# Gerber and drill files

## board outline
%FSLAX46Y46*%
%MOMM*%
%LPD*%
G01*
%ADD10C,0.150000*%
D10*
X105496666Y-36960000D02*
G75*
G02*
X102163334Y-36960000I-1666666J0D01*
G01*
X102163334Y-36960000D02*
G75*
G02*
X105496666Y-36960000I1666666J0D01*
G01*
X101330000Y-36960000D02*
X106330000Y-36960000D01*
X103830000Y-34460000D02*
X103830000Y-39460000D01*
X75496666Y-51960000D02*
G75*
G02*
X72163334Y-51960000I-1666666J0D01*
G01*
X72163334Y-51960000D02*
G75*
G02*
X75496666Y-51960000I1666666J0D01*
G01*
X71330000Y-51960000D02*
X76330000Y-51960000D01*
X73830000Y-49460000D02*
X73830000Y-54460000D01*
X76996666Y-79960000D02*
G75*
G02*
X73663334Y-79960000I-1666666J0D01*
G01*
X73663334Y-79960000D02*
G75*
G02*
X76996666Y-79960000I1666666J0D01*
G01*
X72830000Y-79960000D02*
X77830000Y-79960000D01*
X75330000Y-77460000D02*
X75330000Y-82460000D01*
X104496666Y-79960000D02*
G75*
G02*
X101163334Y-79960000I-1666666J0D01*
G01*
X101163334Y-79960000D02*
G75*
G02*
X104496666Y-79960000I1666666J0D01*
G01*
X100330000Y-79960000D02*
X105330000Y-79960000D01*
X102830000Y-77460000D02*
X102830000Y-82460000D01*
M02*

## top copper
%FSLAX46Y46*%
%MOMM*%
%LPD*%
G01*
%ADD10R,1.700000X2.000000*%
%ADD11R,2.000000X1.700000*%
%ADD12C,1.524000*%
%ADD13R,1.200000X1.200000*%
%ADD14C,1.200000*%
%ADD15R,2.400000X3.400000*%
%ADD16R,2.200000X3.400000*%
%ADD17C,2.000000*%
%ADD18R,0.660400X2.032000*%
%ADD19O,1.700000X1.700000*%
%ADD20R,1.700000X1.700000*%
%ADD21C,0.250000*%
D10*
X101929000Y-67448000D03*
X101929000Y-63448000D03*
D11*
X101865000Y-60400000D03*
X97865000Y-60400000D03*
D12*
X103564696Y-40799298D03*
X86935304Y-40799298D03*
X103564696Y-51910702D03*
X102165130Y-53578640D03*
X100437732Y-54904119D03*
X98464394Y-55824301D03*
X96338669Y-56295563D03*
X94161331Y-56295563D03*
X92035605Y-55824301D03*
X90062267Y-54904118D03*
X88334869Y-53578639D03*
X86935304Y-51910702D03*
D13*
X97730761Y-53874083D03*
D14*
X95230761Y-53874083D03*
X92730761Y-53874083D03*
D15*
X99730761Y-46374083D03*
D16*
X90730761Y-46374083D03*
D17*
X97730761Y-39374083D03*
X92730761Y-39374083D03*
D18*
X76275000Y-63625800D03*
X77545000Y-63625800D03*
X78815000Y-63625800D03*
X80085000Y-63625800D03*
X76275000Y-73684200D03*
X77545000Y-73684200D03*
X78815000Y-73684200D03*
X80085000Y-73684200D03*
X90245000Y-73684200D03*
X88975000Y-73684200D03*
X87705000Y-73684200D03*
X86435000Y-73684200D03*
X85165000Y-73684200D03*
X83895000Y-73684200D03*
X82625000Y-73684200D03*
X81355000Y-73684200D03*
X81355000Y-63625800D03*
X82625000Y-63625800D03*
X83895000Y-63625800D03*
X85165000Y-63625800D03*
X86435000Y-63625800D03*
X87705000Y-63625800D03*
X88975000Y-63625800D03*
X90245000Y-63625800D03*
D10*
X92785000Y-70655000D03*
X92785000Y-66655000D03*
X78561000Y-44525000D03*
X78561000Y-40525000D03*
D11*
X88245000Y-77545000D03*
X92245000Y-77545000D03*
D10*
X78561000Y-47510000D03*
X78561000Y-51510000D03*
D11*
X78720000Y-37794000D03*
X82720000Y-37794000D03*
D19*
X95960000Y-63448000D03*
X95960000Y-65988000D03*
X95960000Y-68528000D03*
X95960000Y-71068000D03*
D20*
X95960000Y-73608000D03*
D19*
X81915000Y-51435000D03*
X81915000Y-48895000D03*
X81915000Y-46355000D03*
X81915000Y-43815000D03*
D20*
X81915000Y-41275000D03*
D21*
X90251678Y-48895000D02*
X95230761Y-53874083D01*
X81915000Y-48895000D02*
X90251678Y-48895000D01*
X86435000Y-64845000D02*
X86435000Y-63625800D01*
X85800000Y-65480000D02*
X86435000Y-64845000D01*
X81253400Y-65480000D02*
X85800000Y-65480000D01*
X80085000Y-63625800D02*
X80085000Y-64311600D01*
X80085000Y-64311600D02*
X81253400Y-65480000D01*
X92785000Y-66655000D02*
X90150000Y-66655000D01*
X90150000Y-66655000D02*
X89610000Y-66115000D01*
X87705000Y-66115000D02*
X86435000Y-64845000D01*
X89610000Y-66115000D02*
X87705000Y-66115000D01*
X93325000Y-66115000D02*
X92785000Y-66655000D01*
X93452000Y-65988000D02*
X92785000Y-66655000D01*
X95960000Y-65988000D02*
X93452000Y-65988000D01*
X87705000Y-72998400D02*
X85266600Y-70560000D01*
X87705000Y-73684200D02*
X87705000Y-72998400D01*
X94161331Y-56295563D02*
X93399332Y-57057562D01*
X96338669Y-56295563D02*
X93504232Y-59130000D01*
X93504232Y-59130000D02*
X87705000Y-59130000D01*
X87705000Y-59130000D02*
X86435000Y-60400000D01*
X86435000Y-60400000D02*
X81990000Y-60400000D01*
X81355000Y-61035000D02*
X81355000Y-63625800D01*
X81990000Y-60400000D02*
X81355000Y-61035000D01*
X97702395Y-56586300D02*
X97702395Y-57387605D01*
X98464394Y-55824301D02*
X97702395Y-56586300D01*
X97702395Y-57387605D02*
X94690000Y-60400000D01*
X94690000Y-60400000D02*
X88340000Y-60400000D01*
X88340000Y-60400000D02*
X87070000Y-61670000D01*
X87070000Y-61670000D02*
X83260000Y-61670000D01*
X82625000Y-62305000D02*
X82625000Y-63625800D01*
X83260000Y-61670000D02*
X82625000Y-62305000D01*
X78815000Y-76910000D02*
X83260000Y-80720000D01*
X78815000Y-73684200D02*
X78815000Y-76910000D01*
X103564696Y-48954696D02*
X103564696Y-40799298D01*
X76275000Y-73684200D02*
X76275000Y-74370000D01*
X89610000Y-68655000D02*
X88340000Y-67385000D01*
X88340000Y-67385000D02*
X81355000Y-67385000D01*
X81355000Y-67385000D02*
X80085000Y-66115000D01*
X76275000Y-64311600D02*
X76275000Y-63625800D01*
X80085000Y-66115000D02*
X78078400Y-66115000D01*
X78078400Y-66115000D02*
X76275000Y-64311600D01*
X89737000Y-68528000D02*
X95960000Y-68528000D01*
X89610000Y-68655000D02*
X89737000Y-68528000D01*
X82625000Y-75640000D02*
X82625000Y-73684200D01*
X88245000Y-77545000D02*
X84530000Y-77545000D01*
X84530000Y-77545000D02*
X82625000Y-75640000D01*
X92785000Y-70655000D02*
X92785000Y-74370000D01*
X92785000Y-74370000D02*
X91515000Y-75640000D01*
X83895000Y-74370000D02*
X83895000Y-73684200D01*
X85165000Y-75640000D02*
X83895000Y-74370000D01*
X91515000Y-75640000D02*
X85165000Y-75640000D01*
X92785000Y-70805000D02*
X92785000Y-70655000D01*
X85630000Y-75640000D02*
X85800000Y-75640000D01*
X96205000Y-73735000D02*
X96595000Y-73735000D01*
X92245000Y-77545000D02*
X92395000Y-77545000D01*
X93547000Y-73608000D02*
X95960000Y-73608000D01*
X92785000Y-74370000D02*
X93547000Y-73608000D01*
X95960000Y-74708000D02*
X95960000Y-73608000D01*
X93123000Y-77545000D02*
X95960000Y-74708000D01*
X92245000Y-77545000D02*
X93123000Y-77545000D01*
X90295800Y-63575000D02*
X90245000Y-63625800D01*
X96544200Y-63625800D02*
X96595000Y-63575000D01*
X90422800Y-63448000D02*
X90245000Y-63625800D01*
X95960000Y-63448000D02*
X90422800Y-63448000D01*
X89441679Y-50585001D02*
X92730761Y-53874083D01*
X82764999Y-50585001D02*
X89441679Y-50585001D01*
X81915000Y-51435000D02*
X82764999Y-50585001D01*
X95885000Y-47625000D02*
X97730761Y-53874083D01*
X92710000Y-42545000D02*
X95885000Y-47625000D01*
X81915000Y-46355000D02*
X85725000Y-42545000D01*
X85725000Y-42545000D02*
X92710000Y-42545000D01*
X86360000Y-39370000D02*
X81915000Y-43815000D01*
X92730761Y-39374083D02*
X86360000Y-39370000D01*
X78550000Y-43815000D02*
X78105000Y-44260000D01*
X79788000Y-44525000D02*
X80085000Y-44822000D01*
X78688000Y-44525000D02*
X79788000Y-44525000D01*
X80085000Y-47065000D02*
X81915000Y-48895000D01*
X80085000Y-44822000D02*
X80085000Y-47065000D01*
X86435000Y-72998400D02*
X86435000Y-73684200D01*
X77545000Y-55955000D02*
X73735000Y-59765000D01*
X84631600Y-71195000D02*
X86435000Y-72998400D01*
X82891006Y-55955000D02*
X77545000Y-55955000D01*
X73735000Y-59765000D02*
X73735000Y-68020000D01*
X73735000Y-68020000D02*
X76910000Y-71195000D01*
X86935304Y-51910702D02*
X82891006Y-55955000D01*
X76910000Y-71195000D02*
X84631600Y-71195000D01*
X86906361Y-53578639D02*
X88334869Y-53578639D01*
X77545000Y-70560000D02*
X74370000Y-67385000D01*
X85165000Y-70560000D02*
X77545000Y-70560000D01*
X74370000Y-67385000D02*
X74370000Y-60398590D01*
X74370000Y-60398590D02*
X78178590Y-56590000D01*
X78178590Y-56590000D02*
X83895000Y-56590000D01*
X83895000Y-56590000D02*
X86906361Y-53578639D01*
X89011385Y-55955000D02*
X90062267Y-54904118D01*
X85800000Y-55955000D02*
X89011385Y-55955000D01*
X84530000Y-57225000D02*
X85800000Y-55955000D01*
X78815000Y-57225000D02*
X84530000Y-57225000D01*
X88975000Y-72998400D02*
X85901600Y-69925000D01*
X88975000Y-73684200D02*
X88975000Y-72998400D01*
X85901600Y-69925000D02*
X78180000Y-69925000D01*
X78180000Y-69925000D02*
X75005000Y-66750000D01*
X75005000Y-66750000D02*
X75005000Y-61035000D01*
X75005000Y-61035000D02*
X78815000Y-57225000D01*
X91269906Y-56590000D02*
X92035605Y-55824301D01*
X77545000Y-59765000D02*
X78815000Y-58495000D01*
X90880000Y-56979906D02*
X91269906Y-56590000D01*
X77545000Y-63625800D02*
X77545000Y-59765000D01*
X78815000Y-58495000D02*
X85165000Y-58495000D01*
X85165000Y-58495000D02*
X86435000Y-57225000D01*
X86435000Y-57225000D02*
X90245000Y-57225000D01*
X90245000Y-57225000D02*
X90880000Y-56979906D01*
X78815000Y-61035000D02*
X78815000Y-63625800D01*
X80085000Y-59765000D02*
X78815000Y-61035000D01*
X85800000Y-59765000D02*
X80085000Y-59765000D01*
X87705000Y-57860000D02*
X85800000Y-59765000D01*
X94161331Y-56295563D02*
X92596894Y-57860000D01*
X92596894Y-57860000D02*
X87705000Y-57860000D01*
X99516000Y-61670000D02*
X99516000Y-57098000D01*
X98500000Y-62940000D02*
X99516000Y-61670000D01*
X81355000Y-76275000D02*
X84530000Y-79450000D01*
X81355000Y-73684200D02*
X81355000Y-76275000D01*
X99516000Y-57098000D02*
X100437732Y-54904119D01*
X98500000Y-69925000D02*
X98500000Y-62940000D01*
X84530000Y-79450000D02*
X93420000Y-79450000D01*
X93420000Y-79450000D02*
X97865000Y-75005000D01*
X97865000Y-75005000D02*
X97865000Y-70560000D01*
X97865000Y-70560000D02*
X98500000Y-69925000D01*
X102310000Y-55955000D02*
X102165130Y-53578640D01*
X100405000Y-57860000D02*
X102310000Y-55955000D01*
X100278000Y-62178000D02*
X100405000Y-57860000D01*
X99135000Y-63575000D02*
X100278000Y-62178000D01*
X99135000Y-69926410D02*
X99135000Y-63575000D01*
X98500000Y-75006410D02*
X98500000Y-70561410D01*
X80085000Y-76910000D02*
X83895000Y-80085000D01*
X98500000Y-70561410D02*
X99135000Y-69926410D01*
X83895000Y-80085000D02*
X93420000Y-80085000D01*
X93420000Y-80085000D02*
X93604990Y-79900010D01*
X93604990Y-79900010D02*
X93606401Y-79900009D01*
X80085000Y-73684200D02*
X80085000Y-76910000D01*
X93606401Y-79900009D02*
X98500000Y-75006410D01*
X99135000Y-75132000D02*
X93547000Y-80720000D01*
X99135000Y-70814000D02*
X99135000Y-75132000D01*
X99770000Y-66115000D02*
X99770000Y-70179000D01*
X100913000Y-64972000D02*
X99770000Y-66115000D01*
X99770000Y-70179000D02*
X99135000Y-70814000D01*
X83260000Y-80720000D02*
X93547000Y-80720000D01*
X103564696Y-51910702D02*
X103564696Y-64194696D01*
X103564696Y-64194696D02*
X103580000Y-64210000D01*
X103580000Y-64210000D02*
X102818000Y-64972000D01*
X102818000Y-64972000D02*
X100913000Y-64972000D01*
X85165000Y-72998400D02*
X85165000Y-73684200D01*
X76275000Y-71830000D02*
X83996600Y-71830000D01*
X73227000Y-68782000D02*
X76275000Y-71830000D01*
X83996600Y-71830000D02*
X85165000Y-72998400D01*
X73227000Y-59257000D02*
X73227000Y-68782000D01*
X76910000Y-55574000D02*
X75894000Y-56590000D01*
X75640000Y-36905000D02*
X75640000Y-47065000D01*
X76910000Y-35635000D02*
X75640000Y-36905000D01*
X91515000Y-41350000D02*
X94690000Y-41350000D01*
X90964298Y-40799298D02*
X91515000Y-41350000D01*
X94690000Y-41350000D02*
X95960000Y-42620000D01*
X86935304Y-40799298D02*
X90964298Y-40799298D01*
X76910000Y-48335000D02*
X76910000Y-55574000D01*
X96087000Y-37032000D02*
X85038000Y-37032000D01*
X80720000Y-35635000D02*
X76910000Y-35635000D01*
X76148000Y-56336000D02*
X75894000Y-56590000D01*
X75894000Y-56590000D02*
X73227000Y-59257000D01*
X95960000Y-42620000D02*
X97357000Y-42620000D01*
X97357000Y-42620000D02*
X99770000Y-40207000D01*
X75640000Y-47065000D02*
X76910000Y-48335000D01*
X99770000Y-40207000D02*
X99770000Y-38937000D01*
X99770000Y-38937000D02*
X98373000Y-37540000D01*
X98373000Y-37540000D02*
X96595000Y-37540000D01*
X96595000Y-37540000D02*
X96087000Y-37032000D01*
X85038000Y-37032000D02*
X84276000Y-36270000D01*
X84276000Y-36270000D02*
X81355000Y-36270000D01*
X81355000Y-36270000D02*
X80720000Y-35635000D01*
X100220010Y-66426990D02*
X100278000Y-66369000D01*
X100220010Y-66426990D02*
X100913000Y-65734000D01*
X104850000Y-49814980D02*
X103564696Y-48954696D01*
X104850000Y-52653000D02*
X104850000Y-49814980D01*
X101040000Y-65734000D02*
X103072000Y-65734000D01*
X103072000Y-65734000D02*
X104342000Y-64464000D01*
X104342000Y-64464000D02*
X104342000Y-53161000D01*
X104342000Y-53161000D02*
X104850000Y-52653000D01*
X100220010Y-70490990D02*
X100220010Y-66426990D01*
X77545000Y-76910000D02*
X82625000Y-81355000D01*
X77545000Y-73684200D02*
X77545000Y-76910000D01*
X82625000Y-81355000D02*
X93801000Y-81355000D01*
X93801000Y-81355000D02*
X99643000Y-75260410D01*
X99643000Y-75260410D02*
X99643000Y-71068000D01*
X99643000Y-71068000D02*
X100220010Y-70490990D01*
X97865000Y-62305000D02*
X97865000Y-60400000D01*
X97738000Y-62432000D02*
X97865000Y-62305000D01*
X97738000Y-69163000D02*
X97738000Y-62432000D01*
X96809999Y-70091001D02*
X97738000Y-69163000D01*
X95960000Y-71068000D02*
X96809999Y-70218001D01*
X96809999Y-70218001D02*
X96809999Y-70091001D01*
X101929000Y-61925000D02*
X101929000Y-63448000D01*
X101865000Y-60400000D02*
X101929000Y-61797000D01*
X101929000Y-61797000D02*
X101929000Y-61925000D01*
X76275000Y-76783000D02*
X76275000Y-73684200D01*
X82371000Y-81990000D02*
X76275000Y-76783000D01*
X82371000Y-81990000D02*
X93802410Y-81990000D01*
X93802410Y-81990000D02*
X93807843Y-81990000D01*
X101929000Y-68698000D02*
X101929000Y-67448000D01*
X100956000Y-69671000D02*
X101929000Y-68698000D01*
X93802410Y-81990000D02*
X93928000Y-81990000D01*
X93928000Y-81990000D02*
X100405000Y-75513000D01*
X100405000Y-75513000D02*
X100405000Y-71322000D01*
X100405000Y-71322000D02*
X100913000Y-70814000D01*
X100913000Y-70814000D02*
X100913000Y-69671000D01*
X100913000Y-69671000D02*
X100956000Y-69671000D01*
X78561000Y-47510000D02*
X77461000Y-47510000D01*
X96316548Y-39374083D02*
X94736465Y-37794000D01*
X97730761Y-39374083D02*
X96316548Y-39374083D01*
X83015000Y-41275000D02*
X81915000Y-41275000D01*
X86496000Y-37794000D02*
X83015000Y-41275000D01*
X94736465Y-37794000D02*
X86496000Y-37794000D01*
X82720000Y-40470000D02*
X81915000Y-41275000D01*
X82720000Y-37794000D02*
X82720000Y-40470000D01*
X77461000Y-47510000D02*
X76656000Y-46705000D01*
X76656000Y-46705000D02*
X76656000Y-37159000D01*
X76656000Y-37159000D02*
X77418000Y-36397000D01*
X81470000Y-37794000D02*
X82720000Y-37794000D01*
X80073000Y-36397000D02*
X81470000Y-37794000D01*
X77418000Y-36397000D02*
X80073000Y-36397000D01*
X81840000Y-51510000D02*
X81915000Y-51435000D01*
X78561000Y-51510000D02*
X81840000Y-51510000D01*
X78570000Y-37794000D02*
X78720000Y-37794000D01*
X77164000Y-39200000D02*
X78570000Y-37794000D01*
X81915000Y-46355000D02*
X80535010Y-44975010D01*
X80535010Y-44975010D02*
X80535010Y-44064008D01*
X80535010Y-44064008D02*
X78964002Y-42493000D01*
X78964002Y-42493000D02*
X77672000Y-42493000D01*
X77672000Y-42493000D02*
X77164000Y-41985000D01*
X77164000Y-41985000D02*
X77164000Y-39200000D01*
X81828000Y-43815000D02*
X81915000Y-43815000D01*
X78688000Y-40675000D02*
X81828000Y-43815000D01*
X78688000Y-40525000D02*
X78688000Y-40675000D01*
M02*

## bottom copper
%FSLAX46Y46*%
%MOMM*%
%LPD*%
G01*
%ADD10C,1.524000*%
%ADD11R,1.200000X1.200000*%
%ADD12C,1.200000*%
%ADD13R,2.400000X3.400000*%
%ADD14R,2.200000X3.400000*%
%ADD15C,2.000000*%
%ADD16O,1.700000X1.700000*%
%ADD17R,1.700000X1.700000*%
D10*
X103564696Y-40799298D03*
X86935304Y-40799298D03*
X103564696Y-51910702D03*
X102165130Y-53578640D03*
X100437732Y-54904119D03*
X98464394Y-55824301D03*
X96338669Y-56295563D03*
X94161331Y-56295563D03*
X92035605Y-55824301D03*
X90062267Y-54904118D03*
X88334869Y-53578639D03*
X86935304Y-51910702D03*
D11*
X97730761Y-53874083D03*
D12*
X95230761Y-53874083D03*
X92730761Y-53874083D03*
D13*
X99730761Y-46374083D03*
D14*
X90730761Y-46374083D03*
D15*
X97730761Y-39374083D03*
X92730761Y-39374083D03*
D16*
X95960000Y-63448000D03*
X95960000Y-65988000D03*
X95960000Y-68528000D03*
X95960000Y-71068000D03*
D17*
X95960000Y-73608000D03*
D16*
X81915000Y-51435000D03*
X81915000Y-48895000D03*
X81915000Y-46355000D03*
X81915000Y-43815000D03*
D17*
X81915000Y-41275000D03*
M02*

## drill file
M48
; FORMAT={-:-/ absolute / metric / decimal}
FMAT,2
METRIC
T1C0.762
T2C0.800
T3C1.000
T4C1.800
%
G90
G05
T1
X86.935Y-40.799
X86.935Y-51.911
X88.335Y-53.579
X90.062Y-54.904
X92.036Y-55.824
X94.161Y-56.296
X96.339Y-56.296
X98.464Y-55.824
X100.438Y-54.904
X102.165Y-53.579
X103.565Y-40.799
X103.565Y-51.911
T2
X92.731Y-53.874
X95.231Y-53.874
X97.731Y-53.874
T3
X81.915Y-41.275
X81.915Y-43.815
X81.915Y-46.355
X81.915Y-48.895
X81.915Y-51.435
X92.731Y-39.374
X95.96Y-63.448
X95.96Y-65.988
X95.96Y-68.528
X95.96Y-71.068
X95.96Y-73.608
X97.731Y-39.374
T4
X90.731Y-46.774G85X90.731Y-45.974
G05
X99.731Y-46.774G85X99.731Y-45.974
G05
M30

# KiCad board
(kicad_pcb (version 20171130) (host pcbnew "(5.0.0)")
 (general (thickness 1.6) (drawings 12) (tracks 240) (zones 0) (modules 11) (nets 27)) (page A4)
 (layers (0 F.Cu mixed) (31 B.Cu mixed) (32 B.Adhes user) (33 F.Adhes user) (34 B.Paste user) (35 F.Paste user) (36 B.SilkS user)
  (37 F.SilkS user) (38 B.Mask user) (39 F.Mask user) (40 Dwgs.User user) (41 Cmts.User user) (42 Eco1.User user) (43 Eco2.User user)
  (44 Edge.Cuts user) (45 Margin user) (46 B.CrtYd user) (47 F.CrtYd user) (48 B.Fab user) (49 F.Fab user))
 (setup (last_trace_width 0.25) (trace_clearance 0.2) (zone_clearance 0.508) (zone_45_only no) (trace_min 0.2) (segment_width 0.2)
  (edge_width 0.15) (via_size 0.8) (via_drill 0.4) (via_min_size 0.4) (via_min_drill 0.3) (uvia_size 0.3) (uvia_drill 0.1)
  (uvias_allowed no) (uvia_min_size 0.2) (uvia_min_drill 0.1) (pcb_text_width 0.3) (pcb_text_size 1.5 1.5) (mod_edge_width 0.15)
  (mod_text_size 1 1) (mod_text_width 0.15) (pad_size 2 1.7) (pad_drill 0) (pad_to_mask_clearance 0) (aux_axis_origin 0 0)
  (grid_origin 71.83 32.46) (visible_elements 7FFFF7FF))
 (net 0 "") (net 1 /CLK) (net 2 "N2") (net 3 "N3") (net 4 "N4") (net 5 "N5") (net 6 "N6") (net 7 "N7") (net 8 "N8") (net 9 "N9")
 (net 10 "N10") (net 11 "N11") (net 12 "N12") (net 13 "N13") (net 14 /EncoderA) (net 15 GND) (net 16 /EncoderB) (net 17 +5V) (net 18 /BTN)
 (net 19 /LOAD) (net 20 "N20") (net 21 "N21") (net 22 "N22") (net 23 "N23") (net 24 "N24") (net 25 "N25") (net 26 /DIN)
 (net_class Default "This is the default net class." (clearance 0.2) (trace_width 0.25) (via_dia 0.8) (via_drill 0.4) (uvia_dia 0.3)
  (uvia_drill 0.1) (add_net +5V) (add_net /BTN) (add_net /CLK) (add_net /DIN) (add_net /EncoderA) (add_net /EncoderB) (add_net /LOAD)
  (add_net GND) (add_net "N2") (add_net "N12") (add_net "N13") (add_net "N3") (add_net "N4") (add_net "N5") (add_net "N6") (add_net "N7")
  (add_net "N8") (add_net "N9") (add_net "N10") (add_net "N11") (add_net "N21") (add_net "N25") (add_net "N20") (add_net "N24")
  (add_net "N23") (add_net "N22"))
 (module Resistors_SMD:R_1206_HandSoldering (layer F.Cu) (at 101.929 65.448 90)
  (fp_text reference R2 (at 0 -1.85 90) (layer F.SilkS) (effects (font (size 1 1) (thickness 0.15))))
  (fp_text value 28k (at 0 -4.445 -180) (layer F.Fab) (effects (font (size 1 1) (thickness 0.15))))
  (pad 1 smd rect (at -2 0 90) (size 2 1.7) (layers F.Cu F.Paste F.Mask) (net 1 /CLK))
  (pad 2 smd rect (at 2 0 90) (size 2 1.7) (layers F.Cu F.Paste F.Mask) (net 1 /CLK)))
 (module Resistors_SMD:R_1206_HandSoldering (layer F.Cu) (at 99.865 60.4)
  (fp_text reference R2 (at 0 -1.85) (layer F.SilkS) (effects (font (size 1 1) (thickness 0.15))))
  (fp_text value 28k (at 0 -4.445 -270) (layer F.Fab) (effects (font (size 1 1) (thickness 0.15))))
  (pad 2 smd rect (at 2 0) (size 2 1.7) (layers F.Cu F.Paste F.Mask) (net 1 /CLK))
  (pad 1 smd rect (at -2 0) (size 2 1.7) (layers F.Cu F.Paste F.Mask) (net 1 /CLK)))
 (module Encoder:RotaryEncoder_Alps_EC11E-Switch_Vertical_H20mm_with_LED (layer B.Cu) (at 95.25 46.355 180)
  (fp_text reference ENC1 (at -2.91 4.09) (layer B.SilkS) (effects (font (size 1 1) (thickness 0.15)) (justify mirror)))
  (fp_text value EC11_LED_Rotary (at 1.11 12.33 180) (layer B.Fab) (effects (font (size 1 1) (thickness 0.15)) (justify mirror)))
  (pad 1 thru_hole circle (at -8.314696 5.555702 123.8) (size 1.524 1.524) (drill 0.762) (layers *.Cu *.Mask) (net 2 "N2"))
  (pad 12 thru_hole circle (at 8.314696 5.555702 123.8) (size 1.524 1.524) (drill 0.762) (layers *.Cu *.Mask) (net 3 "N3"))
  (pad 2 thru_hole circle (at -8.314696 -5.555702 123.8) (size 1.524 1.524) (drill 0.762) (layers *.Cu *.Mask) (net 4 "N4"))
  (pad 3 thru_hole circle (at -6.91513 -7.22364 123.8) (size 1.524 1.524) (drill 0.762) (layers *.Cu *.Mask) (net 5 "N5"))
  (pad 4 thru_hole circle (at -5.187732 -8.549119 123.8) (size 1.524 1.524) (drill 0.762) (layers *.Cu *.Mask) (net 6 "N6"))
  (pad 5 thru_hole circle (at -3.214394 -9.469301 123.8) (size 1.524 1.524) (drill 0.762) (layers *.Cu *.Mask) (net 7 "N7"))
  (pad 6 thru_hole circle (at -1.088669 -9.940563 123.8) (size 1.524 1.524) (drill 0.762) (layers *.Cu *.Mask) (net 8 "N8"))
  (pad 7 thru_hole circle (at 1.088669 -9.940563 123.8) (size 1.524 1.524) (drill 0.762) (layers *.Cu *.Mask) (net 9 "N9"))
  (pad 8 thru_hole circle (at 3.214395 -9.469301 123.8) (size 1.524 1.524) (drill 0.762) (layers *.Cu *.Mask) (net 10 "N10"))
  (pad 9 thru_hole circle (at 5.187733 -8.549118 123.8) (size 1.524 1.524) (drill 0.762) (layers *.Cu *.Mask) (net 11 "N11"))
  (pad 10 thru_hole circle (at 6.915131 -7.223639 123.8) (size 1.524 1.524) (drill 0.762) (layers *.Cu *.Mask) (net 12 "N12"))
  (pad 11 thru_hole circle (at 8.314696 -5.555702 123.8) (size 1.524 1.524) (drill 0.762) (layers *.Cu *.Mask) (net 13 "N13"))
  (pad A thru_hole rect (at -2.480761 -7.519083 90) (size 1.2 1.2) (drill 0.8) (layers *.Cu *.Mask) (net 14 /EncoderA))
  (pad C thru_hole circle (at 0.019239 -7.519083 90) (size 1.2 1.2) (drill 0.8) (layers *.Cu *.Mask) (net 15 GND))
  (pad B thru_hole circle (at 2.519239 -7.519083 90) (size 1.2 1.2) (drill 0.8) (layers *.Cu *.Mask) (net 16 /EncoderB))
  (pad MP thru_hole rect (at -4.480761 -0.019083 90) (size 3.4 2.4) (drill oval 2.6 1.8) (layers *.Cu *.Mask))
  (pad MP thru_hole rect (at 4.519239 -0.019083 90) (size 3.4 2.2) (drill oval 2.6 1.8) (layers *.Cu *.Mask))
  (pad SW2 thru_hole circle (at -2.480761 6.980917 90) (size 2 2) (drill 1) (layers *.Cu *.Mask) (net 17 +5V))
  (pad SW1 thru_hole circle (at 2.519239 6.980917 90) (size 2 2) (drill 1) (layers *.Cu *.Mask) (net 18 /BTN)))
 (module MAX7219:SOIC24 (layer F.Cu) (at 83.26 68.655 180)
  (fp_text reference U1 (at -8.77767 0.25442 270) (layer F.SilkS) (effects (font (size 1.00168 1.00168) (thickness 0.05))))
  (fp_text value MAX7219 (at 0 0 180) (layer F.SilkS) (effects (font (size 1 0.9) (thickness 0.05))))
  (pad 12 smd rect (at 6.985 5.0292 180) (size 0.6604 2.032) (layers F.Cu F.Paste F.Mask) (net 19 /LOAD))
  (pad 11 smd rect (at 5.715 5.0292 180) (size 0.6604 2.032) (layers F.Cu F.Paste F.Mask) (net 10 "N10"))
  (pad 10 smd rect (at 4.445 5.0292 180) (size 0.6604 2.032) (layers F.Cu F.Paste F.Mask) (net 9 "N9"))
  (pad 9 smd rect (at 3.175 5.0292 180) (size 0.6604 2.032) (layers F.Cu F.Paste F.Mask) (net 15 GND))
  (pad 13 smd rect (at 6.985 -5.0292 180) (size 0.6604 2.032) (layers F.Cu F.Paste F.Mask) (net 1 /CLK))
  (pad 14 smd rect (at 5.715 -5.0292 180) (size 0.6604 2.032) (layers F.Cu F.Paste F.Mask) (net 2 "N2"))
  (pad 15 smd rect (at 4.445 -5.0292 180) (size 0.6604 2.032) (layers F.Cu F.Paste F.Mask) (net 4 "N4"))
  (pad 16 smd rect (at 3.175 -5.0292 180) (size 0.6604 2.032) (layers F.Cu F.Paste F.Mask) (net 5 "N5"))
  (pad 24 smd rect (at -6.985 -5.0292 180) (size 0.6604 2.032) (layers F.Cu F.Paste F.Mask) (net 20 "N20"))
  (pad 23 smd rect (at -5.715 -5.0292 180) (size 0.6604 2.032) (layers F.Cu F.Paste F.Mask) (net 11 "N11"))
  (pad 22 smd rect (at -4.445 -5.0292 180) (size 0.6604 2.032) (layers F.Cu F.Paste F.Mask) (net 12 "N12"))
  (pad 21 smd rect (at -3.175 -5.0292 180) (size 0.6604 2.032) (layers F.Cu F.Paste F.Mask) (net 13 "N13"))
  (pad 20 smd rect (at -1.905 -5.0292 180) (size 0.6604 2.032) (layers F.Cu F.Paste F.Mask) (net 3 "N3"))
  (pad 19 smd rect (at -0.635 -5.0292 180) (size 0.6604 2.032) (layers F.Cu F.Paste F.Mask) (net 17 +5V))
  (pad 18 smd rect (at 0.635 -5.0292 180) (size 0.6604 2.032) (layers F.Cu F.Paste F.Mask) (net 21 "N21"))
  (pad 17 smd rect (at 1.905 -5.0292 180) (size 0.6604 2.032) (layers F.Cu F.Paste F.Mask) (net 6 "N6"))
  (pad 8 smd rect (at 1.905 5.0292 180) (size 0.6604 2.032) (layers F.Cu F.Paste F.Mask) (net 8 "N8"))
  (pad 7 smd rect (at 0.635 5.0292 180) (size 0.6604 2.032) (layers F.Cu F.Paste F.Mask) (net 7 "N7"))
  (pad 6 smd rect (at -0.635 5.0292 180) (size 0.6604 2.032) (layers F.Cu F.Paste F.Mask) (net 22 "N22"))
  (pad 5 smd rect (at -1.905 5.0292 180) (size 0.6604 2.032) (layers F.Cu F.Paste F.Mask) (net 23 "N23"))
  (pad 4 smd rect (at -3.175 5.0292 180) (size 0.6604 2.032) (layers F.Cu F.Paste F.Mask) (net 15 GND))
  (pad 3 smd rect (at -4.445 5.0292 180) (size 0.6604 2.032) (layers F.Cu F.Paste F.Mask) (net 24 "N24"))
  (pad 2 smd rect (at -5.715 5.0292 180) (size 0.6604 2.032) (layers F.Cu F.Paste F.Mask) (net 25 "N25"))
  (pad 1 smd rect (at -6.985 5.0292 180) (size 0.6604 2.032) (layers F.Cu F.Paste F.Mask) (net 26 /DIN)))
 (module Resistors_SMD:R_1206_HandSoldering (layer F.Cu) (at 92.785 68.655 90)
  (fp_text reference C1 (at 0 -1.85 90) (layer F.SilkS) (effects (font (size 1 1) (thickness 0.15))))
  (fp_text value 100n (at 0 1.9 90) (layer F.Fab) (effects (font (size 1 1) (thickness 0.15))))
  (pad 1 smd rect (at -2 0 90) (size 2 1.7) (layers F.Cu F.Paste F.Mask) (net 17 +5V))
  (pad 2 smd rect (at 2 0 90) (size 2 1.7) (layers F.Cu F.Paste F.Mask) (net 15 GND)))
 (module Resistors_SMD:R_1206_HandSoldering (layer F.Cu) (at 78.561 42.525 90)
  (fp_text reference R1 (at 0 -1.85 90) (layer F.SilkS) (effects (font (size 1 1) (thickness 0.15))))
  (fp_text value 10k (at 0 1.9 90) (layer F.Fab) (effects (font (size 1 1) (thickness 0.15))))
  (pad 1 smd rect (at -2 0 90) (size 2 1.7) (layers F.Cu F.Paste F.Mask) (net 15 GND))
  (pad 2 smd rect (at 2 0 90) (size 2 1.7) (layers F.Cu F.Paste F.Mask) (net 18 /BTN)))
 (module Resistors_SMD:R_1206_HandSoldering (layer F.Cu) (at 90.245 77.545)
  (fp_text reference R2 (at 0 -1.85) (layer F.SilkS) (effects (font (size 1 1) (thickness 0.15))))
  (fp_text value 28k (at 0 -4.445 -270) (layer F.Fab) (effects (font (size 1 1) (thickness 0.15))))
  (pad 1 smd rect (at -2 0) (size 2 1.7) (layers F.Cu F.Paste F.Mask) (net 21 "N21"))
  (pad 2 smd rect (at 2 0) (size 2 1.7) (layers F.Cu F.Paste F.Mask) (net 17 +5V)))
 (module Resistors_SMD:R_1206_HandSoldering (layer F.Cu) (at 78.561 49.51 270)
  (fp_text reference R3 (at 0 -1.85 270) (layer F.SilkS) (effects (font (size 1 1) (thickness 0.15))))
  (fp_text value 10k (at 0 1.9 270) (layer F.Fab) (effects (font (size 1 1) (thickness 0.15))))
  (pad 1 smd rect (at -2 0 270) (size 2 1.7) (layers F.Cu F.Paste F.Mask) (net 17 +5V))
  (pad 2 smd rect (at 2 0 270) (size 2 1.7) (layers F.Cu F.Paste F.Mask) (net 16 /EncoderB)))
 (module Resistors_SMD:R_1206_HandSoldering (layer F.Cu) (at 80.72 37.794)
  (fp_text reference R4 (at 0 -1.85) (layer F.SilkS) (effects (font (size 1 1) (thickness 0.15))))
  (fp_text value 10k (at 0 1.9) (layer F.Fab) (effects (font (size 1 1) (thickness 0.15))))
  (pad 1 smd rect (at -2 0) (size 2 1.7) (layers F.Cu F.Paste F.Mask) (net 14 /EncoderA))
  (pad 2 smd rect (at 2 0) (size 2 1.7) (layers F.Cu F.Paste F.Mask) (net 17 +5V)))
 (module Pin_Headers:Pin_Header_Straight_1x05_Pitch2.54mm (layer F.Cu) (at 95.96 73.608 180)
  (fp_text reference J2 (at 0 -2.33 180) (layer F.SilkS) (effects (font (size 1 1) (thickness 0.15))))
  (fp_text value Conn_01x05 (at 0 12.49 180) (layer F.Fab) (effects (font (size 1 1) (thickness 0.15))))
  (pad 5 thru_hole oval (at 0 10.16 180) (size 1.7 1.7) (drill 1) (layers *.Cu *.Mask) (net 26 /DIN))
  (pad 4 thru_hole oval (at 0 7.62 180) (size 1.7 1.7) (drill 1) (layers *.Cu *.Mask) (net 15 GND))
  (pad 3 thru_hole oval (at 0 5.08 180) (size 1.7 1.7) (drill 1) (layers *.Cu *.Mask) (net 19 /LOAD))
  (pad 2 thru_hole oval (at 0 2.54 180) (size 1.7 1.7) (drill 1) (layers *.Cu *.Mask) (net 1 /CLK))
  (pad 1 thru_hole rect (at 0 0 180) (size 1.7 1.7) (drill 1) (layers *.Cu *.Mask) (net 17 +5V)))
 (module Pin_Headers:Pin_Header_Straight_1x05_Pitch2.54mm (layer F.Cu) (at 81.915 41.275)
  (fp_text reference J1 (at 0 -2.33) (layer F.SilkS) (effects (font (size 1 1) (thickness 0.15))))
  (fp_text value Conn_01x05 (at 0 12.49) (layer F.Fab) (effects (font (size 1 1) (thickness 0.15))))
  (pad 5 thru_hole oval (at 0 10.16) (size 1.7 1.7) (drill 1) (layers *.Cu *.Mask) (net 16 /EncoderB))
  (pad 4 thru_hole oval (at 0 7.62) (size 1.7 1.7) (drill 1) (layers *.Cu *.Mask) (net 15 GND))
  (pad 3 thru_hole oval (at 0 5.08) (size 1.7 1.7) (drill 1) (layers *.Cu *.Mask) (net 14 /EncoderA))
  (pad 2 thru_hole oval (at 0 2.54) (size 1.7 1.7) (drill 1) (layers *.Cu *.Mask) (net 18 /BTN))
  (pad 1 thru_hole rect (at 0 0) (size 1.7 1.7) (drill 1) (layers *.Cu *.Mask) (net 17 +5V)))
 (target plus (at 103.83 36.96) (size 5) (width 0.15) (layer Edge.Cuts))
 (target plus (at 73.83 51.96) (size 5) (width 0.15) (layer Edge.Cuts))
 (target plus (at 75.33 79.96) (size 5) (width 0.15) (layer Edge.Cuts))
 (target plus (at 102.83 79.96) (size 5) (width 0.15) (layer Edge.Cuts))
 (segment (start 90.251678 48.895) (end 95.230761 53.874083) (width 0.25) (layer F.Cu) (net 15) (status 20))
 (segment (start 81.915 48.895) (end 90.251678 48.895) (width 0.25) (layer F.Cu) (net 15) (status 10))
 (segment (start 86.435 64.845) (end 86.435 63.6258) (width 0.25) (layer F.Cu) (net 15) (status 20))
 (segment (start 85.8 65.48) (end 86.435 64.845) (width 0.25) (layer F.Cu) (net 15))
 (segment (start 81.2534 65.48) (end 85.8 65.48) (width 0.25) (layer F.Cu) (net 15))
 (segment (start 80.085 63.6258) (end 80.085 64.3116) (width 0.25) (layer F.Cu) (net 15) (status 30))
 (segment (start 80.085 64.3116) (end 81.2534 65.48) (width 0.25) (layer F.Cu) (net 15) (status 10))
 (segment (start 92.785 66.655) (end 90.15 66.655) (width 0.25) (layer F.Cu) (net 15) (status 10))
 (segment (start 90.15 66.655) (end 89.61 66.115) (width 0.25) (layer F.Cu) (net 15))
 (segment (start 87.705 66.115) (end 86.435 64.845) (width 0.25) (layer F.Cu) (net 15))
 (segment (start 89.61 66.115) (end 87.705 66.115) (width 0.25) (layer F.Cu) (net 15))
 (segment (start 93.325 66.115) (end 92.785 66.655) (width 0.25) (layer F.Cu) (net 15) (status 30))
 (segment (start 93.452 65.988) (end 92.785 66.655) (width 0.25) (layer F.Cu) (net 15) (status 30))
 (segment (start 95.96 65.988) (end 93.452 65.988) (width 0.25) (layer F.Cu) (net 15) (status 30))
 (segment (start 87.705 72.9984) (end 85.2666 70.56) (width 0.25) (layer F.Cu) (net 12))
 (segment (start 87.705 73.6842) (end 87.705 72.9984) (width 0.25) (layer F.Cu) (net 12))
 (segment (start 94.161331 56.295563) (end 93.399332 57.057562) (width 0.25) (layer F.Cu) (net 9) (status 10))
 (segment (start 96.338669 56.295563) (end 93.504232 59.13) (width 0.25) (layer F.Cu) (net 8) (status 10))
 (segment (start 93.504232 59.13) (end 87.705 59.13) (width 0.25) (layer F.Cu) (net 8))
 (segment (start 87.705 59.13) (end 86.435 60.4) (width 0.25) (layer F.Cu) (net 8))
 (segment (start 86.435 60.4) (end 81.99 60.4) (width 0.25) (layer F.Cu) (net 8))
 (segment (start 81.355 61.035) (end 81.355 63.6258) (width 0.25) (layer F.Cu) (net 8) (status 20))
 (segment (start 81.99 60.4) (end 81.355 61.035) (width 0.25) (layer F.Cu) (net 8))
 (segment (start 97.702395 56.5863) (end 97.702395 57.387605) (width 0.25) (layer F.Cu) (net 7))
 (segment (start 98.464394 55.824301) (end 97.702395 56.5863) (width 0.25) (layer F.Cu) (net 7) (status 10))
 (segment (start 97.702395 57.387605) (end 94.69 60.4) (width 0.25) (layer F.Cu) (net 7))
 (segment (start 94.69 60.4) (end 88.34 60.4) (width 0.25) (layer F.Cu) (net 7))
 (segment (start 88.34 60.4) (end 87.07 61.67) (width 0.25) (layer F.Cu) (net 7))
 (segment (start 87.07 61.67) (end 83.26 61.67) (width 0.25) (layer F.Cu) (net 7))
 (segment (start 82.625 62.305) (end 82.625 63.6258) (width 0.25) (layer F.Cu) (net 7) (status 20))
 (segment (start 83.26 61.67) (end 82.625 62.305) (width 0.25) (layer F.Cu) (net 7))
 (segment (start 78.815 76.91) (end 83.26 80.72) (width 0.25) (layer F.Cu) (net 4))
 (segment (start 78.815 73.6842) (end 78.815 76.91) (width 0.25) (layer F.Cu) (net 4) (status 10))
 (segment (start 103.564696 48.954696) (end 103.564696 40.799298) (width 0.25) (layer F.Cu) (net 2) (status 20))
 (segment (start 76.275 73.6842) (end 76.275 74.37) (width 0.25) (layer F.Cu) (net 1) (status 30))
 (segment (start 89.61 68.655) (end 88.34 67.385) (width 0.25) (layer F.Cu) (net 19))
 (segment (start 88.34 67.385) (end 81.355 67.385) (width 0.25) (layer F.Cu) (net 19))
 (segment (start 81.355 67.385) (end 80.085 66.115) (width 0.25) (layer F.Cu) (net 19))
 (segment (start 76.275 64.3116) (end 76.275 63.6258) (width 0.25) (layer F.Cu) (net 19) (status 30))
 (segment (start 80.085 66.115) (end 78.0784 66.115) (width 0.25) (layer F.Cu) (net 19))
 (segment (start 78.0784 66.115) (end 76.275 64.3116) (width 0.25) (layer F.Cu) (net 19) (status 20))
 (segment (start 89.737 68.528) (end 95.96 68.528) (width 0.25) (layer F.Cu) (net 19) (status 20))
 (segment (start 89.61 68.655) (end 89.737 68.528) (width 0.25) (layer F.Cu) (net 19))
 (segment (start 82.625 75.64) (end 82.625 73.6842) (width 0.25) (layer F.Cu) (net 21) (status 20))
 (segment (start 88.245 77.545) (end 84.53 77.545) (width 0.25) (layer F.Cu) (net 21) (status 10))
 (segment (start 84.53 77.545) (end 82.625 75.64) (width 0.25) (layer F.Cu) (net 21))
 (segment (start 92.785 70.655) (end 92.785 74.37) (width 0.25) (layer F.Cu) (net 17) (status 10))
 (segment (start 92.785 74.37) (end 91.515 75.64) (width 0.25) (layer F.Cu) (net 17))
 (segment (start 83.895 74.37) (end 83.895 73.6842) (width 0.25) (layer F.Cu) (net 17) (status 30))
 (segment (start 85.165 75.64) (end 83.895 74.37) (width 0.25) (layer F.Cu) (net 17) (status 20))
 (segment (start 91.515 75.64) (end 85.165 75.64) (width 0.25) (layer F.Cu) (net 17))
 (segment (start 92.785 70.805) (end 92.785 70.655) (width 0.25) (layer F.Cu) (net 17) (status 30))
 (segment (start 85.63 75.64) (end 85.8 75.64) (width 0.25) (layer F.Cu) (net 17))
 (segment (start 96.205 73.735) (end 96.595 73.735) (width 0.25) (layer F.Cu) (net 17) (status 30))
 (segment (start 92.245 77.545) (end 92.395 77.545) (width 0.25) (layer F.Cu) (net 17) (status 30))
 (segment (start 93.547 73.608) (end 95.96 73.608) (width 0.25) (layer F.Cu) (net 17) (status 20))
 (segment (start 92.785 74.37) (end 93.547 73.608) (width 0.25) (layer F.Cu) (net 17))
 (segment (start 95.96 74.708) (end 95.96 73.608) (width 0.25) (layer F.Cu) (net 17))
 (segment (start 93.123 77.545) (end 95.96 74.708) (width 0.25) (layer F.Cu) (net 17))
 (segment (start 92.245 77.545) (end 93.123 77.545) (width 0.25) (layer F.Cu) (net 17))
 (segment (start 90.2958 63.575) (end 90.245 63.6258) (width 0.25) (layer F.Cu) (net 26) (status 30))
 (segment (start 96.5442 63.6258) (end 96.595 63.575) (width 0.25) (layer F.Cu) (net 26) (status 30))
 (segment (start 90.4228 63.448) (end 90.245 63.6258) (width 0.25) (layer F.Cu) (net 26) (status 30))
 (segment (start 95.96 63.448) (end 90.4228 63.448) (width 0.25) (layer F.Cu) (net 26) (status 30))
 (segment (start 89.441679 50.585001) (end 92.730761 53.874083) (width 0.25) (layer F.Cu) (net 16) (status 20))
 (segment (start 82.764999 50.585001) (end 89.441679 50.585001) (width 0.25) (layer F.Cu) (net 16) (status 10))
 (segment (start 81.915 51.435) (end 82.764999 50.585001) (width 0.25) (layer F.Cu) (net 16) (status 30))
 (segment (start 95.885 47.625) (end 97.730761 53.874083) (width 0.25) (layer F.Cu) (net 14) (status 20))
 (segment (start 92.71 42.545) (end 95.885 47.625) (width 0.25) (layer F.Cu) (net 14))
 (segment (start 81.915 46.355) (end 85.725 42.545) (width 0.25) (layer F.Cu) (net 14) (status 10))
 (segment (start 85.725 42.545) (end 92.71 42.545) (width 0.25) (layer F.Cu) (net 14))
 (segment (start 86.36 39.37) (end 81.915 43.815) (width 0.25) (layer F.Cu) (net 18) (status 20))
 (segment (start 92.730761 39.374083) (end 86.36 39.37) (width 0.25) (layer F.Cu) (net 18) (status 10))
 (segment (start 78.55 43.815) (end 78.105 44.26) (width 0.25) (layer F.Cu) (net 15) (status 30))
 (segment (start 79.788 44.525) (end 80.085 44.822) (width 0.25) (layer F.Cu) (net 15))
 (segment (start 78.688 44.525) (end 79.788 44.525) (width 0.25) (layer F.Cu) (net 15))
 (segment (start 80.085 47.065) (end 81.915 48.895) (width 0.25) (layer F.Cu) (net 15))
 (segment (start 80.085 44.822) (end 80.085 47.065) (width 0.25) (layer F.Cu) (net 15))
 (segment (start 86.435 72.9984) (end 86.435 73.6842) (width 0.25) (layer F.Cu) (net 13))
 (segment (start 77.545 55.955) (end 73.735 59.765) (width 0.25) (layer F.Cu) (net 13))
 (segment (start 84.6316 71.195) (end 86.435 72.9984) (width 0.25) (layer F.Cu) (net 13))
 (segment (start 82.891006 55.955) (end 77.545 55.955) (width 0.25) (layer F.Cu) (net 13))
 (segment (start 73.735 59.765) (end 73.735 68.02) (width 0.25) (layer F.Cu) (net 13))
 (segment (start 73.735 68.02) (end 76.91 71.195) (width 0.25) (layer F.Cu) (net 13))
 (segment (start 86.935304 51.910702) (end 82.891006 55.955) (width 0.25) (layer F.Cu) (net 13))
 (segment (start 76.91 71.195) (end 84.6316 71.195) (width 0.25) (layer F.Cu) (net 13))
 (segment (start 86.906361 53.578639) (end 88.334869 53.578639) (width 0.25) (layer F.Cu) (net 12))
 (segment (start 77.545 70.56) (end 74.37 67.385) (width 0.25) (layer F.Cu) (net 12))
 (segment (start 85.165 70.56) (end 77.545 70.56) (width 0.25) (layer F.Cu) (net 12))
 (segment (start 74.37 67.385) (end 74.37 60.39859) (width 0.25) (layer F.Cu) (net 12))
 (segment (start 74.37 60.39859) (end 78.17859 56.59) (width 0.25) (layer F.Cu) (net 12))
 (segment (start 78.17859 56.59) (end 83.895 56.59) (width 0.25) (layer F.Cu) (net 12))
 (segment (start 83.895 56.59) (end 86.906361 53.578639) (width 0.25) (layer F.Cu) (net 12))
 (segment (start 89.011385 55.955) (end 90.062267 54.904118) (width 0.25) (layer F.Cu) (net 11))
 (segment (start 85.8 55.955) (end 89.011385 55.955) (width 0.25) (layer F.Cu) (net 11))
 (segment (start 84.53 57.225) (end 85.8 55.955) (width 0.25) (layer F.Cu) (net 11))
 (segment (start 78.815 57.225) (end 84.53 57.225) (width 0.25) (layer F.Cu) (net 11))
 (segment (start 88.975 72.9984) (end 85.9016 69.925) (width 0.25) (layer F.Cu) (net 11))
 (segment (start 88.975 73.6842) (end 88.975 72.9984) (width 0.25) (layer F.Cu) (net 11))
 (segment (start 85.9016 69.925) (end 78.18 69.925) (width 0.25) (layer F.Cu) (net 11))
 (segment (start 78.18 69.925) (end 75.005 66.75) (width 0.25) (layer F.Cu) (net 11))
 (segment (start 75.005 66.75) (end 75.005 61.035) (width 0.25) (layer F.Cu) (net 11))
 (segment (start 75.005 61.035) (end 78.815 57.225) (width 0.25) (layer F.Cu) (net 11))
 (segment (start 91.269906 56.59) (end 92.035605 55.824301) (width 0.25) (layer F.Cu) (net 10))
 (segment (start 77.545 59.765) (end 78.815 58.495) (width 0.25) (layer F.Cu) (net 10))
 (segment (start 90.88 56.979906) (end 91.269906 56.59) (width 0.25) (layer F.Cu) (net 10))
 (segment (start 77.545 63.6258) (end 77.545 59.765) (width 0.25) (layer F.Cu) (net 10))
 (segment (start 78.815 58.495) (end 85.165 58.495) (width 0.25) (layer F.Cu) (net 10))
 (segment (start 85.165 58.495) (end 86.435 57.225) (width 0.25) (layer F.Cu) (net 10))
 (segment (start 86.435 57.225) (end 90.245 57.225) (width 0.25) (layer F.Cu) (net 10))
 (segment (start 90.245 57.225) (end 90.88 56.979906) (width 0.25) (layer F.Cu) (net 10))
 (segment (start 78.815 61.035) (end 78.815 63.6258) (width 0.25) (layer F.Cu) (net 9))
 (segment (start 80.085 59.765) (end 78.815 61.035) (width 0.25) (layer F.Cu) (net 9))
 (segment (start 85.8 59.765) (end 80.085 59.765) (width 0.25) (layer F.Cu) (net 9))
 (segment (start 87.705 57.86) (end 85.8 59.765) (width 0.25) (layer F.Cu) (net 9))
 (segment (start 94.161331 56.295563) (end 92.596894 57.86) (width 0.25) (layer F.Cu) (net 9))
 (segment (start 92.596894 57.86) (end 87.705 57.86) (width 0.25) (layer F.Cu) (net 9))
 (segment (start 99.516 61.67) (end 99.516 57.098) (width 0.25) (layer F.Cu) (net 6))
 (segment (start 98.5 62.94) (end 99.516 61.67) (width 0.25) (layer F.Cu) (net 6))
 (segment (start 81.355 76.275) (end 84.53 79.45) (width 0.25) (layer F.Cu) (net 6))
 (segment (start 81.355 73.6842) (end 81.355 76.275) (width 0.25) (layer F.Cu) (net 6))
 (segment (start 99.516 57.098) (end 100.437732 54.904119) (width 0.25) (layer F.Cu) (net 6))
 (segment (start 98.5 69.925) (end 98.5 62.94) (width 0.25) (layer F.Cu) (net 6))
 (segment (start 84.53 79.45) (end 93.42 79.45) (width 0.25) (layer F.Cu) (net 6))
 (segment (start 93.42 79.45) (end 97.865 75.005) (width 0.25) (layer F.Cu) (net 6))
 (segment (start 97.865 75.005) (end 97.865 70.56) (width 0.25) (layer F.Cu) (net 6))
 (segment (start 97.865 70.56) (end 98.5 69.925) (width 0.25) (layer F.Cu) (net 6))
 (segment (start 102.31 55.955) (end 102.16513 53.57864) (width 0.25) (layer F.Cu) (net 5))
 (segment (start 100.405 57.86) (end 102.31 55.955) (width 0.25) (layer F.Cu) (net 5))
 (segment (start 100.278 62.178) (end 100.405 57.86) (width 0.25) (layer F.Cu) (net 5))
 (segment (start 99.135 63.575) (end 100.278 62.178) (width 0.25) (layer F.Cu) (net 5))
 (segment (start 99.135 69.92641) (end 99.135 63.575) (width 0.25) (layer F.Cu) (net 5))
 (segment (start 98.5 75.00641) (end 98.5 70.56141) (width 0.25) (layer F.Cu) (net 5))
 (segment (start 80.085 76.91) (end 83.895 80.085) (width 0.25) (layer F.Cu) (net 5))
 (segment (start 98.5 70.56141) (end 99.135 69.92641) (width 0.25) (layer F.Cu) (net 5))
 (segment (start 83.895 80.085) (end 93.42 80.085) (width 0.25) (layer F.Cu) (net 5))
 (segment (start 93.42 80.085) (end 93.60499 79.90001) (width 0.25) (layer F.Cu) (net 5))
 (segment (start 93.60499 79.90001) (end 93.606401 79.900009) (width 0.25) (layer F.Cu) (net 5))
 (segment (start 80.085 73.6842) (end 80.085 76.91) (width 0.25) (layer F.Cu) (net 5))
 (segment (start 93.606401 79.900009) (end 98.5 75.00641) (width 0.25) (layer F.Cu) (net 5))
 (segment (start 99.135 75.132) (end 93.547 80.72) (width 0.25) (layer F.Cu) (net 4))
 (segment (start 99.135 70.814) (end 99.135 75.132) (width 0.25) (layer F.Cu) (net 4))
 (segment (start 99.77 66.115) (end 99.77 70.179) (width 0.25) (layer F.Cu) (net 4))
 (segment (start 100.913 64.972) (end 99.77 66.115) (width 0.25) (layer F.Cu) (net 4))
 (segment (start 99.77 70.179) (end 99.135 70.814) (width 0.25) (layer F.Cu) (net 4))
 (segment (start 83.26 80.72) (end 93.547 80.72) (width 0.25) (layer F.Cu) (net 4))
 (segment (start 103.564696 51.910702) (end 103.564696 64.194696) (width 0.25) (layer F.Cu) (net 4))
 (segment (start 103.564696 64.194696) (end 103.58 64.21) (width 0.25) (layer F.Cu) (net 4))
 (segment (start 103.58 64.21) (end 102.818 64.972) (width 0.25) (layer F.Cu) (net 4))
 (segment (start 102.818 64.972) (end 100.913 64.972) (width 0.25) (layer F.Cu) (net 4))
 (segment (start 85.165 72.9984) (end 85.165 73.6842) (width 0.25) (layer F.Cu) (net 3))
 (segment (start 76.275 71.83) (end 83.9966 71.83) (width 0.25) (layer F.Cu) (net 3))
 (segment (start 73.227 68.782) (end 76.275 71.83) (width 0.25) (layer F.Cu) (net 3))
 (segment (start 83.9966 71.83) (end 85.165 72.9984) (width 0.25) (layer F.Cu) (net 3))
 (segment (start 73.227 59.257) (end 73.227 68.782) (width 0.25) (layer F.Cu) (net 3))
 (segment (start 76.91 55.574) (end 75.894 56.59) (width 0.25) (layer F.Cu) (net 3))
 (segment (start 75.64 36.905) (end 75.64 47.065) (width 0.25) (layer F.Cu) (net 3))
 (segment (start 76.91 35.635) (end 75.64 36.905) (width 0.25) (layer F.Cu) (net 3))
 (segment (start 91.515 41.35) (end 94.69 41.35) (width 0.25) (layer F.Cu) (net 3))
 (segment (start 90.964298 40.799298) (end 91.515 41.35) (width 0.25) (layer F.Cu) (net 3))
 (segment (start 94.69 41.35) (end 95.96 42.62) (width 0.25) (layer F.Cu) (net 3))
 (segment (start 86.935304 40.799298) (end 90.964298 40.799298) (width 0.25) (layer F.Cu) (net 3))
 (segment (start 76.91 48.335) (end 76.91 55.574) (width 0.25) (layer F.Cu) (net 3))
 (segment (start 96.087 37.032) (end 85.038 37.032) (width 0.25) (layer F.Cu) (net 3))
 (segment (start 80.72 35.635) (end 76.91 35.635) (width 0.25) (layer F.Cu) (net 3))
 (segment (start 76.148 56.336) (end 75.894 56.59) (width 0.25) (layer F.Cu) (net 3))
 (segment (start 75.894 56.59) (end 73.227 59.257) (width 0.25) (layer F.Cu) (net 3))
 (segment (start 95.96 42.62) (end 97.357 42.62) (width 0.25) (layer F.Cu) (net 3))
 (segment (start 97.357 42.62) (end 99.77 40.207) (width 0.25) (layer F.Cu) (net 3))
 (segment (start 75.64 47.065) (end 76.91 48.335) (width 0.25) (layer F.Cu) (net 3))
 (segment (start 99.77 40.207) (end 99.77 38.937) (width 0.25) (layer F.Cu) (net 3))
 (segment (start 99.77 38.937) (end 98.373 37.54) (width 0.25) (layer F.Cu) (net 3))
 (segment (start 98.373 37.54) (end 96.595 37.54) (width 0.25) (layer F.Cu) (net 3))
 (segment (start 96.595 37.54) (end 96.087 37.032) (width 0.25) (layer F.Cu) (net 3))
 (segment (start 85.038 37.032) (end 84.276 36.27) (width 0.25) (layer F.Cu) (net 3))
 (segment (start 84.276 36.27) (end 81.355 36.27) (width 0.25) (layer F.Cu) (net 3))
 (segment (start 81.355 36.27) (end 80.72 35.635) (width 0.25) (layer F.Cu) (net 3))
 (segment (start 100.22001 66.42699) (end 100.278 66.369) (width 0.25) (layer F.Cu) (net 2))
 (segment (start 100.22001 66.42699) (end 100.913 65.734) (width 0.25) (layer F.Cu) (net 2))
 (segment (start 104.85 49.81498) (end 103.564696 48.954696) (width 0.25) (layer F.Cu) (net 2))
 (segment (start 104.85 52.653) (end 104.85 49.81498) (width 0.25) (layer F.Cu) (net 2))
 (segment (start 101.04 65.734) (end 103.072 65.734) (width 0.25) (layer F.Cu) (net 2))
 (segment (start 103.072 65.734) (end 104.342 64.464) (width 0.25) (layer F.Cu) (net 2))
 (segment (start 104.342 64.464) (end 104.342 53.161) (width 0.25) (layer F.Cu) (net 2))
 (segment (start 104.342 53.161) (end 104.85 52.653) (width 0.25) (layer F.Cu) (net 2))
 (segment (start 100.22001 70.49099) (end 100.22001 66.42699) (width 0.25) (layer F.Cu) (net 2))
 (segment (start 77.545 76.91) (end 82.625 81.355) (width 0.25) (layer F.Cu) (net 2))
 (segment (start 77.545 73.6842) (end 77.545 76.91) (width 0.25) (layer F.Cu) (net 2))
 (segment (start 82.625 81.355) (end 93.801 81.355) (width 0.25) (layer F.Cu) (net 2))
 (segment (start 93.801 81.355) (end 99.643 75.26041) (width 0.25) (layer F.Cu) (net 2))
 (segment (start 99.643 75.26041) (end 99.643 71.068) (width 0.25) (layer F.Cu) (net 2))
 (segment (start 99.643 71.068) (end 100.22001 70.49099) (width 0.25) (layer F.Cu) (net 2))
 (segment (start 97.865 62.305) (end 97.865 60.4) (width 0.25) (layer F.Cu) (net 1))
 (segment (start 97.738 62.432) (end 97.865 62.305) (width 0.25) (layer F.Cu) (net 1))
 (segment (start 97.738 69.163) (end 97.738 62.432) (width 0.25) (layer F.Cu) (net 1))
 (segment (start 96.809999 70.091001) (end 97.738 69.163) (width 0.25) (layer F.Cu) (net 1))
 (segment (start 95.96 71.068) (end 96.809999 70.218001) (width 0.25) (layer F.Cu) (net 1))
 (segment (start 96.809999 70.218001) (end 96.809999 70.091001) (width 0.25) (layer F.Cu) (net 1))
 (segment (start 101.929 61.925) (end 101.929 63.448) (width 0.25) (layer F.Cu) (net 1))
 (segment (start 101.865 60.4) (end 101.929 61.797) (width 0.25) (layer F.Cu) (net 1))
 (segment (start 101.929 61.797) (end 101.929 61.925) (width 0.25) (layer F.Cu) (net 1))
 (segment (start 76.275 76.783) (end 76.275 73.6842) (width 0.25) (layer F.Cu) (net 1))
 (segment (start 82.371 81.99) (end 76.275 76.783) (width 0.25) (layer F.Cu) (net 1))
 (segment (start 82.371 81.99) (end 93.80241 81.99) (width 0.25) (layer F.Cu) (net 1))
 (segment (start 93.80241 81.99) (end 93.807843 81.99) (width 0.25) (layer F.Cu) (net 1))
 (segment (start 101.929 68.698) (end 101.929 67.448) (width 0.25) (layer F.Cu) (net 1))
 (segment (start 100.956 69.671) (end 101.929 68.698) (width 0.25) (layer F.Cu) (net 1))
 (segment (start 93.80241 81.99) (end 93.928 81.99) (width 0.25) (layer F.Cu) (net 1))
 (segment (start 93.928 81.99) (end 100.405 75.513) (width 0.25) (layer F.Cu) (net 1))
 (segment (start 100.405 75.513) (end 100.405 71.322) (width 0.25) (layer F.Cu) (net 1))
 (segment (start 100.405 71.322) (end 100.913 70.814) (width 0.25) (layer F.Cu) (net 1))
 (segment (start 100.913 70.814) (end 100.913 69.671) (width 0.25) (layer F.Cu) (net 1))
 (segment (start 100.913 69.671) (end 100.956 69.671) (width 0.25) (layer F.Cu) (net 1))
 (segment (start 78.561 47.51) (end 77.461 47.51) (width 0.25) (layer F.Cu) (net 17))
 (segment (start 96.316548 39.374083) (end 94.736465 37.794) (width 0.25) (layer F.Cu) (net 17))
 (segment (start 97.730761 39.374083) (end 96.316548 39.374083) (width 0.25) (layer F.Cu) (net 17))
 (segment (start 83.015 41.275) (end 81.915 41.275) (width 0.25) (layer F.Cu) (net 17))
 (segment (start 86.496 37.794) (end 83.015 41.275) (width 0.25) (layer F.Cu) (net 17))
 (segment (start 94.736465 37.794) (end 86.496 37.794) (width 0.25) (layer F.Cu) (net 17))
 (segment (start 82.72 40.47) (end 81.915 41.275) (width 0.25) (layer F.Cu) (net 17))
 (segment (start 82.72 37.794) (end 82.72 40.47) (width 0.25) (layer F.Cu) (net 17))
 (segment (start 77.461 47.51) (end 76.656 46.705) (width 0.25) (layer F.Cu) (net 17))
 (segment (start 76.656 46.705) (end 76.656 37.159) (width 0.25) (layer F.Cu) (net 17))
 (segment (start 76.656 37.159) (end 77.418 36.397) (width 0.25) (layer F.Cu) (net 17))
 (segment (start 81.47 37.794) (end 82.72 37.794) (width 0.25) (layer F.Cu) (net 17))
 (segment (start 80.073 36.397) (end 81.47 37.794) (width 0.25) (layer F.Cu) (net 17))
 (segment (start 77.418 36.397) (end 80.073 36.397) (width 0.25) (layer F.Cu) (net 17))
 (segment (start 81.84 51.51) (end 81.915 51.435) (width 0.25) (layer F.Cu) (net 16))
 (segment (start 78.561 51.51) (end 81.84 51.51) (width 0.25) (layer F.Cu) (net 16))
 (segment (start 78.57 37.794) (end 78.72 37.794) (width 0.25) (layer F.Cu) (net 14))
 (segment (start 77.164 39.2) (end 78.57 37.794) (width 0.25) (layer F.Cu) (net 14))
 (segment (start 81.915 46.355) (end 80.53501 44.97501) (width 0.25) (layer F.Cu) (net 14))
 (segment (start 80.53501 44.97501) (end 80.53501 44.064008) (width 0.25) (layer F.Cu) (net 14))
 (segment (start 80.53501 44.064008) (end 78.964002 42.493) (width 0.25) (layer F.Cu) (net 14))
 (segment (start 78.964002 42.493) (end 77.672 42.493) (width 0.25) (layer F.Cu) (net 14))
 (segment (start 77.672 42.493) (end 77.164 41.985) (width 0.25) (layer F.Cu) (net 14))
 (segment (start 77.164 41.985) (end 77.164 39.2) (width 0.25) (layer F.Cu) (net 14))
 (segment (start 81.828 43.815) (end 81.915 43.815) (width 0.25) (layer F.Cu) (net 18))
 (segment (start 78.688 40.675) (end 81.828 43.815) (width 0.25) (layer F.Cu) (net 18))
 (segment (start 78.688 40.525) (end 78.688 40.675) (width 0.25) (layer F.Cu) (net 18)))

